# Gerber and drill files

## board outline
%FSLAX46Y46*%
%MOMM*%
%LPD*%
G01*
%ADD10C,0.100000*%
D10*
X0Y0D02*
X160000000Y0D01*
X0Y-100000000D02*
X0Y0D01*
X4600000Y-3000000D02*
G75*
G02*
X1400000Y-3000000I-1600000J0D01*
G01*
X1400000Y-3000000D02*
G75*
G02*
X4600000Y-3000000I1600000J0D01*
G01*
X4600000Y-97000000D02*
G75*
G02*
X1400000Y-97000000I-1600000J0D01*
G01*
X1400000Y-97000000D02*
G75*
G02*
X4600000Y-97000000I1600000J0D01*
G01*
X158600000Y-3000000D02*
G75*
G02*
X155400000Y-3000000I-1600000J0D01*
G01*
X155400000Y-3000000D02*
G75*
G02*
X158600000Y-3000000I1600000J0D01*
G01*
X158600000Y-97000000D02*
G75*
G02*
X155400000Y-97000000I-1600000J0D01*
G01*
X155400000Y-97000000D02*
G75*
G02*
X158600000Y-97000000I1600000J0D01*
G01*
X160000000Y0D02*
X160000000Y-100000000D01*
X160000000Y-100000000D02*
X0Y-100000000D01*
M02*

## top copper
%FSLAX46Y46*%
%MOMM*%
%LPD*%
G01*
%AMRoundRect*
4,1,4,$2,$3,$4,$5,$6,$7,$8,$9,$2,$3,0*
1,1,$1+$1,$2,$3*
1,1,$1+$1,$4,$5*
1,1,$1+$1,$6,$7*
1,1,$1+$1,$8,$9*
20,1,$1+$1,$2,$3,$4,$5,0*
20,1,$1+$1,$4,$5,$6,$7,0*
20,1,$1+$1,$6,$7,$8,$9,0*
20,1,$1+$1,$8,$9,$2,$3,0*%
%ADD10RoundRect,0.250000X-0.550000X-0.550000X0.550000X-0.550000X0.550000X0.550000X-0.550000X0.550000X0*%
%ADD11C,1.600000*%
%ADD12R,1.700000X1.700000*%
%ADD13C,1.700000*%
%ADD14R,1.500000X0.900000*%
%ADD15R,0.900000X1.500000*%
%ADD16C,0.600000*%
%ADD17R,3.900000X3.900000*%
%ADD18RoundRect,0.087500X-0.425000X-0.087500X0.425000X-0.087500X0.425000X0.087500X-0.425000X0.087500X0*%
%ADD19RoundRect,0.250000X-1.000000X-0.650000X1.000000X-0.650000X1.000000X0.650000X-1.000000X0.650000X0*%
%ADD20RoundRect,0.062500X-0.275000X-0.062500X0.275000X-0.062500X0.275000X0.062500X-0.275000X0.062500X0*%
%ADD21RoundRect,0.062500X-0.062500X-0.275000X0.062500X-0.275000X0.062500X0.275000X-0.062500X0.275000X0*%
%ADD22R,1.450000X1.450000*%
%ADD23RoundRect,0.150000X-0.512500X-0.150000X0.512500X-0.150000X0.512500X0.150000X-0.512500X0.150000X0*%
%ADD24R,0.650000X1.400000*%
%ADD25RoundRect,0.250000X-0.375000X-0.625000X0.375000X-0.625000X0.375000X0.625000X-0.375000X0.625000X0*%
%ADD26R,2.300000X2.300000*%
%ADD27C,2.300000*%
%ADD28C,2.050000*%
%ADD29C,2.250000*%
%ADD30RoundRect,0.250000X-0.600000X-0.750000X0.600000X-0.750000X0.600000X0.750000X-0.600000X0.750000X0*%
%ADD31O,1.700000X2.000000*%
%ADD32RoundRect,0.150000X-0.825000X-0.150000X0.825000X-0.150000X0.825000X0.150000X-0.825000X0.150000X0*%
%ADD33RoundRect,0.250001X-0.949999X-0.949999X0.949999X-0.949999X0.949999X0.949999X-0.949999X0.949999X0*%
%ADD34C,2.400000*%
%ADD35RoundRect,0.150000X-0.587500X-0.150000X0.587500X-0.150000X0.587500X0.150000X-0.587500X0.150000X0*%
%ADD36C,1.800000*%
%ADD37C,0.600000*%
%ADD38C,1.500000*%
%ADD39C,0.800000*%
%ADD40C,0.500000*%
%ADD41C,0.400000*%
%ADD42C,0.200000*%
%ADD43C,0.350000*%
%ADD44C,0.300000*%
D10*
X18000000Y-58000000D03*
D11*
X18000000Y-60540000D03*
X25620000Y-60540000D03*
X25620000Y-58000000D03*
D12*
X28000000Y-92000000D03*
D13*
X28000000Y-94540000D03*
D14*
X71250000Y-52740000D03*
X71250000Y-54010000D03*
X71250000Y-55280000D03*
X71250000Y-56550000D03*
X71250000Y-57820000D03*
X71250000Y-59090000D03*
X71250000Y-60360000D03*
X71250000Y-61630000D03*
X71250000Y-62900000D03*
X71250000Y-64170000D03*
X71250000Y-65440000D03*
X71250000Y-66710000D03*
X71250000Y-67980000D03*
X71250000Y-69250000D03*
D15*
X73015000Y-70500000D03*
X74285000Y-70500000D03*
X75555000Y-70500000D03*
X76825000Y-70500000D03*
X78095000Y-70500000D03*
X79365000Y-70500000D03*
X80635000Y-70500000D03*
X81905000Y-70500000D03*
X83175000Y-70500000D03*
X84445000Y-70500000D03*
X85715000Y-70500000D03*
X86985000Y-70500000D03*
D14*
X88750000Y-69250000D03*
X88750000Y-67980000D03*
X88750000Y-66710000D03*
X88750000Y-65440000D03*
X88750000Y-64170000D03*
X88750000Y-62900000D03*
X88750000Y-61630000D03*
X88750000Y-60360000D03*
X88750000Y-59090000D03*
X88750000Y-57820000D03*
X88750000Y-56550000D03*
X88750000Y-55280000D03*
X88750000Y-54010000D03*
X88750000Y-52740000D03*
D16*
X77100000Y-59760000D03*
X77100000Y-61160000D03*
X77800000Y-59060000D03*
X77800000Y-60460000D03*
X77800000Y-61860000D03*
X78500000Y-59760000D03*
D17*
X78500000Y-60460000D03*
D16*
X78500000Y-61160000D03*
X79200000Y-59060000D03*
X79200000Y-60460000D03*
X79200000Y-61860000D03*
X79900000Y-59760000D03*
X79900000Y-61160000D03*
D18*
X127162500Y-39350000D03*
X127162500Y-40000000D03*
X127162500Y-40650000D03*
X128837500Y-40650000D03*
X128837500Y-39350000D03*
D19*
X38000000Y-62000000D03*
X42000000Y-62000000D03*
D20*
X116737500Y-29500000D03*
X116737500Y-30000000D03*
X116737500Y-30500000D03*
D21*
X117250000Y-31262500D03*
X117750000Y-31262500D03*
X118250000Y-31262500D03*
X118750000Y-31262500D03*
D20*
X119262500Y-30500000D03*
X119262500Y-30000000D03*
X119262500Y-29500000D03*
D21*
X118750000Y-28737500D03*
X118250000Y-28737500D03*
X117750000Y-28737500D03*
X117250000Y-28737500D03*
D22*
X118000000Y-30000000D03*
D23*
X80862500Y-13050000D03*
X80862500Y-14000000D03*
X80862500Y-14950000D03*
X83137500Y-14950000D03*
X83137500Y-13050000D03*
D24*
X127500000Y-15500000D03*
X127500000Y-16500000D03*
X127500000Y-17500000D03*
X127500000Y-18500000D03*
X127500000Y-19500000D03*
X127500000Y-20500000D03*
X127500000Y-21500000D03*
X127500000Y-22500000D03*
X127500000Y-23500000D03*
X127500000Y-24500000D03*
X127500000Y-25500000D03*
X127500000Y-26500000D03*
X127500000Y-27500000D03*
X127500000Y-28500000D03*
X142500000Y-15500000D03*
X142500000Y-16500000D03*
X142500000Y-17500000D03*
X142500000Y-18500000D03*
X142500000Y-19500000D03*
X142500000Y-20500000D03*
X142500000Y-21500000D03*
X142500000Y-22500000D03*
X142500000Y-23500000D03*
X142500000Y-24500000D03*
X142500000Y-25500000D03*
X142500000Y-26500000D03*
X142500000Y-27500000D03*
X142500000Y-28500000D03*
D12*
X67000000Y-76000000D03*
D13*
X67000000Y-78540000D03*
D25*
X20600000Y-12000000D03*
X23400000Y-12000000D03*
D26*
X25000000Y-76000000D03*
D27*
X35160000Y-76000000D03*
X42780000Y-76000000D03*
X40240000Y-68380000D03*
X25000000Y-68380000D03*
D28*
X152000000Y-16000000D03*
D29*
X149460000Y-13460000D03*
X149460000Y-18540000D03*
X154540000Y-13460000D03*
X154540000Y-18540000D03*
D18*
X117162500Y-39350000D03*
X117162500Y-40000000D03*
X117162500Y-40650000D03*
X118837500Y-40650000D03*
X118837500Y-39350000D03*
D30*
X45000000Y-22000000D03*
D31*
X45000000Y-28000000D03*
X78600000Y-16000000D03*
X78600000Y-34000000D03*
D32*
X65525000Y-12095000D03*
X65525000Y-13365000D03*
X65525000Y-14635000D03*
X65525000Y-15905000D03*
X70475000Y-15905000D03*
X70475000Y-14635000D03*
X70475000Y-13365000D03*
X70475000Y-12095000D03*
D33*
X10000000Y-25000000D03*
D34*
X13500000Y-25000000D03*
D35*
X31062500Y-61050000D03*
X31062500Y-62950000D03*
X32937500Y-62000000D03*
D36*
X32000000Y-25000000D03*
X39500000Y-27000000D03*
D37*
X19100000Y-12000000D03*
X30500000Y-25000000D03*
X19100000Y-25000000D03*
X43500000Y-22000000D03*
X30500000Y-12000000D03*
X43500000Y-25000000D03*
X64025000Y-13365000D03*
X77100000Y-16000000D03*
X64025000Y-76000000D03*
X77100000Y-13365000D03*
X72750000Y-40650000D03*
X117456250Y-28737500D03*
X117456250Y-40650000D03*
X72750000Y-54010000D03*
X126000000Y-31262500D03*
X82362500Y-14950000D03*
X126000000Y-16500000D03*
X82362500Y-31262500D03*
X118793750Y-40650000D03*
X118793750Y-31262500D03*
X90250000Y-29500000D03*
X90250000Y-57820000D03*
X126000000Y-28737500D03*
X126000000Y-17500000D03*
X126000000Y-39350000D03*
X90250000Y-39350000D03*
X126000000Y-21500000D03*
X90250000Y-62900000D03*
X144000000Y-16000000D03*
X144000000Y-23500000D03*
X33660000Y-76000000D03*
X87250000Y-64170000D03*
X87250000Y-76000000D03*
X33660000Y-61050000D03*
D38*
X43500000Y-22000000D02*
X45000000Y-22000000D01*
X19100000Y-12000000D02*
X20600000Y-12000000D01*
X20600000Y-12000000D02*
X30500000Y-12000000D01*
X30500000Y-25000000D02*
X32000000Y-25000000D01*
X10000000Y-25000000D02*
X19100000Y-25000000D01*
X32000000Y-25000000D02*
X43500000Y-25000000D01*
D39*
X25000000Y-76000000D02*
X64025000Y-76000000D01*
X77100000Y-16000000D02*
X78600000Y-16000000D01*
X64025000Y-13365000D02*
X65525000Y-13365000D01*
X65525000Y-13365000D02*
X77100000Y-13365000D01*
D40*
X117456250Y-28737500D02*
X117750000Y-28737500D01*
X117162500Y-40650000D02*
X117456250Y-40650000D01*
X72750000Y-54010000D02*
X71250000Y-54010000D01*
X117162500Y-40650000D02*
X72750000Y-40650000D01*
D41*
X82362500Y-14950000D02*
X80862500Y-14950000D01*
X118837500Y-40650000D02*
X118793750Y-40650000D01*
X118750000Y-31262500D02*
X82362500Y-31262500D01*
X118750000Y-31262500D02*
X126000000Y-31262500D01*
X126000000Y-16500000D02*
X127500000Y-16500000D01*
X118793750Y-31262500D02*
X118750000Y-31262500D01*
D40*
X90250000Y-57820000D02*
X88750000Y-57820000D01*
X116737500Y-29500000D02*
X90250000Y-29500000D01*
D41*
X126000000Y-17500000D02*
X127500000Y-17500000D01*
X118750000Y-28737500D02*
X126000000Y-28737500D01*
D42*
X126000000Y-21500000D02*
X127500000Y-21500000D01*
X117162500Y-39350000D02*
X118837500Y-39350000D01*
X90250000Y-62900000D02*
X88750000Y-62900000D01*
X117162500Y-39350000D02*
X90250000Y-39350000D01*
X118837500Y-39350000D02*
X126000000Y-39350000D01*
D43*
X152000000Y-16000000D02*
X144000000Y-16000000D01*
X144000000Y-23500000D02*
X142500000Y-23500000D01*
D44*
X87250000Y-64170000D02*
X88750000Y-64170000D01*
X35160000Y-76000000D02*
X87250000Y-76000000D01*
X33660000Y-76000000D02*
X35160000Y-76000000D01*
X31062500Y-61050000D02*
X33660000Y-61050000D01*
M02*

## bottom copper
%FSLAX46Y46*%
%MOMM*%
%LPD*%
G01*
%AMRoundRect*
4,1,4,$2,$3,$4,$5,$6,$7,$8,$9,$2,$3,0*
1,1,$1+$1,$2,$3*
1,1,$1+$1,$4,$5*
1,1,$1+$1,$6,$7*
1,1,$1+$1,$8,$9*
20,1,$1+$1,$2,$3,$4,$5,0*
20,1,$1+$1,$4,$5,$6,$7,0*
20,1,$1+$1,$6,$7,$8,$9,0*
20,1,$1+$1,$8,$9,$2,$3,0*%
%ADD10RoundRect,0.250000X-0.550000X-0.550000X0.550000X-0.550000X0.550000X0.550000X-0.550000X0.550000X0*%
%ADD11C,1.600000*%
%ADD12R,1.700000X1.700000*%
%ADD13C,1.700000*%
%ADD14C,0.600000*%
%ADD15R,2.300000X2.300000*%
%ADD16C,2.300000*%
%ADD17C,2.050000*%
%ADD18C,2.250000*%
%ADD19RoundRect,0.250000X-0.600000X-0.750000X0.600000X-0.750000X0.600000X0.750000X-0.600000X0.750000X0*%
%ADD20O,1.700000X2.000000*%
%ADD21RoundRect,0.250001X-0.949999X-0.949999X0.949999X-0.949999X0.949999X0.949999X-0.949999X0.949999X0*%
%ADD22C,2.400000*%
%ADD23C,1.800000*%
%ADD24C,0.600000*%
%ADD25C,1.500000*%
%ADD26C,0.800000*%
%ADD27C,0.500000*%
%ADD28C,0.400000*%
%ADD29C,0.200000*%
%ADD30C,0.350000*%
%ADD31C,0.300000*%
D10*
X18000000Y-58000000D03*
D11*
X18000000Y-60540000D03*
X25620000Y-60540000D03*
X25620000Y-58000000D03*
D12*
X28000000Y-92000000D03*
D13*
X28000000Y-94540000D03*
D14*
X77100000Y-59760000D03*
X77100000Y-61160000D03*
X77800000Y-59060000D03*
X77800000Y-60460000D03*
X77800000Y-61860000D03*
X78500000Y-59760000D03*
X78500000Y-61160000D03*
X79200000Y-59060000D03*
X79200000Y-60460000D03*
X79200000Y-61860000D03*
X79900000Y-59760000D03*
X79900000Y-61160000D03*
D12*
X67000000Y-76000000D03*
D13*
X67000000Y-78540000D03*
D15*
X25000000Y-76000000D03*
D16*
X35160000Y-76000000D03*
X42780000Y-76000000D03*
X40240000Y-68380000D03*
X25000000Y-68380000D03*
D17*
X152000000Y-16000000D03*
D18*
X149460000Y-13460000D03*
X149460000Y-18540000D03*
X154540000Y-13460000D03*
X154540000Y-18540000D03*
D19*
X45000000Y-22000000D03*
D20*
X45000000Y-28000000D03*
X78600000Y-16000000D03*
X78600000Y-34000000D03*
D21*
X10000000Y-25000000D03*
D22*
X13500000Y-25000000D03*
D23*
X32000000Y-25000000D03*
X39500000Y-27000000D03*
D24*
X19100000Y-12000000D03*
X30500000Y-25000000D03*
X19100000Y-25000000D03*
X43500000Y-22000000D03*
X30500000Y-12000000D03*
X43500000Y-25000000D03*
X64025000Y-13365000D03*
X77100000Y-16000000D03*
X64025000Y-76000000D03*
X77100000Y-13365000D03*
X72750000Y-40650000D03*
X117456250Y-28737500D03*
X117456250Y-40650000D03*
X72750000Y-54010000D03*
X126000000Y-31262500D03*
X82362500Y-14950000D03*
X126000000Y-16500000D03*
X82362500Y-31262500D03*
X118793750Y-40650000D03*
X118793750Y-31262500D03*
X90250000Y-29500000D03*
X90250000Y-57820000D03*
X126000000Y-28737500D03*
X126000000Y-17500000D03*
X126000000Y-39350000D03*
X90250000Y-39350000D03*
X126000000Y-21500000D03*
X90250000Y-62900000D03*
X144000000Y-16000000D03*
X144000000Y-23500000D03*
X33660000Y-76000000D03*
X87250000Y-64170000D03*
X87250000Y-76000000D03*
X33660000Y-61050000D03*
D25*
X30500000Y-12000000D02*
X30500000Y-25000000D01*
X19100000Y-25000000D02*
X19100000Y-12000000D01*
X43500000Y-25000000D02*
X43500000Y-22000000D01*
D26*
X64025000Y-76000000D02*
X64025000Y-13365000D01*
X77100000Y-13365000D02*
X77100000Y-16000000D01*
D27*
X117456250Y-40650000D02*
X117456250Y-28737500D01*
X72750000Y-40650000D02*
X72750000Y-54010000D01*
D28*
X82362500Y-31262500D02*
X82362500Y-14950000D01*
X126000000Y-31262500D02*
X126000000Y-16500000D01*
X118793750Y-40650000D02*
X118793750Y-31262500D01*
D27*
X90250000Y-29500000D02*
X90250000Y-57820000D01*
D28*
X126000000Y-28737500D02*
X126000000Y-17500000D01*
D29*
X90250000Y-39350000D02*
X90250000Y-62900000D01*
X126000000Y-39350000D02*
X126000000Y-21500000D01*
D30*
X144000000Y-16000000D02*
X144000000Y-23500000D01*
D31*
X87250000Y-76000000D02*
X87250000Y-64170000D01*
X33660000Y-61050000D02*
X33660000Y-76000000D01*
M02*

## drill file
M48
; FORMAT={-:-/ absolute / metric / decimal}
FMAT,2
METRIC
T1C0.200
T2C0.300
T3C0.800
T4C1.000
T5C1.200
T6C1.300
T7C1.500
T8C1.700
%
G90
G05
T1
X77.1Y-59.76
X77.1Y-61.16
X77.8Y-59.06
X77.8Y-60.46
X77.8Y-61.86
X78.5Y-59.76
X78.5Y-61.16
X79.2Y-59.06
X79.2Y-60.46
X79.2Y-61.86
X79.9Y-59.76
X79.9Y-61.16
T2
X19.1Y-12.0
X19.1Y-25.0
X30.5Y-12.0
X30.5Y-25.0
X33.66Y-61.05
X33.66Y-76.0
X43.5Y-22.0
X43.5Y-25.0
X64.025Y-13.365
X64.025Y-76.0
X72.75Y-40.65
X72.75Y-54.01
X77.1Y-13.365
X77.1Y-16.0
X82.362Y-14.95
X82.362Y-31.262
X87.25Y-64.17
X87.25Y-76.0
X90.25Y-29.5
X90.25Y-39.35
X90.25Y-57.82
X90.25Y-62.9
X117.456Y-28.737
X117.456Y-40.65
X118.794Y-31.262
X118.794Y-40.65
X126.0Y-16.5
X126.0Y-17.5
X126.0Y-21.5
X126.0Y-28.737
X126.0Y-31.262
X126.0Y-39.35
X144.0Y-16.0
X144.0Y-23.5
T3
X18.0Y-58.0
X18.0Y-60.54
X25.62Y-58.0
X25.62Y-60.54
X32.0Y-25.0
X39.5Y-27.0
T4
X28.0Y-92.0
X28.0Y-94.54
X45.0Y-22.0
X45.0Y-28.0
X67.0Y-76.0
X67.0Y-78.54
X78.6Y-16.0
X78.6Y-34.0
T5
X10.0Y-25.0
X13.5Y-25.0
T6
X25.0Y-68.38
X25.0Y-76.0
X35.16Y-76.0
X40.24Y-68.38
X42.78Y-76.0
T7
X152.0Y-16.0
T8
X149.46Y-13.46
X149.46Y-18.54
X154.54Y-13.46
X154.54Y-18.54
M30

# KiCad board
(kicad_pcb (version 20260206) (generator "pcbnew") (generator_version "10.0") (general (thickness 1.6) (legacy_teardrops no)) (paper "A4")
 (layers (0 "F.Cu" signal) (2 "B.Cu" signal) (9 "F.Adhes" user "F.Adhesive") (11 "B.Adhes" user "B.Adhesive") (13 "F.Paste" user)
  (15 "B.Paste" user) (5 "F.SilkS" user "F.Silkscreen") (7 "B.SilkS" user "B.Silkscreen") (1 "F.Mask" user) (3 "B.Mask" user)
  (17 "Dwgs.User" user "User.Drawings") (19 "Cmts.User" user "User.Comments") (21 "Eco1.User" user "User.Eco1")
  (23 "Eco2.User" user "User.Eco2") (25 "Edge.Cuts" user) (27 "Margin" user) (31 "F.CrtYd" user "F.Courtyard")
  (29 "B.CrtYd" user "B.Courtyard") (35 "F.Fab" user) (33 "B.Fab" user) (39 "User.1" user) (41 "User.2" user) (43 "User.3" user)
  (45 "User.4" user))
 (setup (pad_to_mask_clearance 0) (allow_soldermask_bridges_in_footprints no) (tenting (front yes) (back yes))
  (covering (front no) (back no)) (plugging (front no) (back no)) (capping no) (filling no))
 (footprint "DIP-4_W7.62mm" (layer "F.Cu") (at 18 58)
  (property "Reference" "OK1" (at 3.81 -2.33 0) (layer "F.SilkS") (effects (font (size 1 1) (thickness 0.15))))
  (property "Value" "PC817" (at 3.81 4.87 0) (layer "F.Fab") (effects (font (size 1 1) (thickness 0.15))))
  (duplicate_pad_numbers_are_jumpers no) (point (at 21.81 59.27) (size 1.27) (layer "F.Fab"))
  (pad "1" thru_hole roundrect (at 0 0) (size 1.6 1.6) (drill 0.8) (layers "*.Cu" "*.Mask") (remove_unused_layers no)
   (roundrect_rratio 0.15625))
  (pad "2" thru_hole circle (at 0 2.54) (size 1.6 1.6) (drill 0.8) (layers "*.Cu" "*.Mask") (remove_unused_layers no))
  (pad "3" thru_hole circle (at 7.62 2.54) (size 1.6 1.6) (drill 0.8) (layers "*.Cu" "*.Mask") (remove_unused_layers no))
  (pad "4" thru_hole circle (at 7.62 0) (size 1.6 1.6) (drill 0.8) (layers "*.Cu" "*.Mask") (remove_unused_layers no)))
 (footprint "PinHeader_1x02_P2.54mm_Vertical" (layer "F.Cu") (at 28 92)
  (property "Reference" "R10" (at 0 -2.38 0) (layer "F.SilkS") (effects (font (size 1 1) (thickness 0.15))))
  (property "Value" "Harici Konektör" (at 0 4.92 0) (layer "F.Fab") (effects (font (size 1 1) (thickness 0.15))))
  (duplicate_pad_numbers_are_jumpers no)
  (pad "1" thru_hole rect (at 0 0) (size 1.7 1.7) (drill 1) (layers "*.Cu" "*.Mask") (remove_unused_layers no))
  (pad "2" thru_hole circle (at 0 2.54) (size 1.7 1.7) (drill 1) (layers "*.Cu" "*.Mask") (remove_unused_layers no)))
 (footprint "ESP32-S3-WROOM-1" (layer "F.Cu") (at 80 58)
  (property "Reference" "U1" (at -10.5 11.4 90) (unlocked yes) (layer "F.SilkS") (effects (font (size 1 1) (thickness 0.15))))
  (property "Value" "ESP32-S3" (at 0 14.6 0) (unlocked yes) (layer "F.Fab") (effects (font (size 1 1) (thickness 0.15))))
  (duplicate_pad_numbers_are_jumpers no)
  (pad "" smd rect (at -2.9 1.06) (size 0.9 0.9) (layers "F.Paste"))
  (pad "" smd rect (at -2.9 2.46 270) (size 0.9 0.9) (layers "F.Paste"))
  (pad "" smd rect (at -2.9 3.86) (size 0.9 0.9) (layers "F.Paste"))
  (pad "" smd rect (at -1.5 1.06 270) (size 0.9 0.9) (layers "F.Paste"))
  (pad "" smd rect (at -1.5 2.46 270) (size 0.9 0.9) (layers "F.Paste"))
  (pad "" smd rect (at -1.5 3.86 270) (size 0.9 0.9) (layers "F.Paste"))
  (pad "" smd rect (at -0.1 1.06 270) (size 0.9 0.9) (layers "F.Paste"))
  (pad "" smd rect (at -0.1 2.46 270) (size 0.9 0.9) (layers "F.Paste"))
  (pad "" smd rect (at -0.1 3.86 270) (size 0.9 0.9) (layers "F.Paste"))
  (pad "1" smd rect (at -8.75 -5.26) (size 1.5 0.9) (layers "F.Cu" "F.Mask" "F.Paste"))
  (pad "2" smd rect (at -8.75 -3.99) (size 1.5 0.9) (layers "F.Cu" "F.Mask" "F.Paste") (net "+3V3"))
  (pad "3" smd rect (at -8.75 -2.72) (size 1.5 0.9) (layers "F.Cu" "F.Mask" "F.Paste"))
  (pad "4" smd rect (at -8.75 -1.45) (size 1.5 0.9) (layers "F.Cu" "F.Mask" "F.Paste"))
  (pad "5" smd rect (at -8.75 -0.18) (size 1.5 0.9) (layers "F.Cu" "F.Mask" "F.Paste"))
  (pad "6" smd rect (at -8.75 1.09) (size 1.5 0.9) (layers "F.Cu" "F.Mask" "F.Paste"))
  (pad "7" smd rect (at -8.75 2.36) (size 1.5 0.9) (layers "F.Cu" "F.Mask" "F.Paste"))
  (pad "8" smd rect (at -8.75 3.63) (size 1.5 0.9) (layers "F.Cu" "F.Mask" "F.Paste"))
  (pad "9" smd rect (at -8.75 4.9) (size 1.5 0.9) (layers "F.Cu" "F.Mask" "F.Paste"))
  (pad "10" smd rect (at -8.75 6.17) (size 1.5 0.9) (layers "F.Cu" "F.Mask" "F.Paste"))
  (pad "11" smd rect (at -8.75 7.44) (size 1.5 0.9) (layers "F.Cu" "F.Mask" "F.Paste"))
  (pad "12" smd rect (at -8.75 8.71) (size 1.5 0.9) (layers "F.Cu" "F.Mask" "F.Paste"))
  (pad "13" smd rect (at -8.75 9.98) (size 1.5 0.9) (layers "F.Cu" "F.Mask" "F.Paste"))
  (pad "14" smd rect (at -8.75 11.25 180) (size 1.5 0.9) (layers "F.Cu" "F.Mask" "F.Paste"))
  (pad "15" smd rect (at -6.985 12.5 270) (size 1.5 0.9) (layers "F.Cu" "F.Mask" "F.Paste"))
  (pad "16" smd rect (at -5.715 12.5 270) (size 1.5 0.9) (layers "F.Cu" "F.Mask" "F.Paste"))
  (pad "17" smd rect (at -4.445 12.5 270) (size 1.5 0.9) (layers "F.Cu" "F.Mask" "F.Paste"))
  (pad "18" smd rect (at -3.175 12.5 270) (size 1.5 0.9) (layers "F.Cu" "F.Mask" "F.Paste"))
  (pad "19" smd rect (at -1.905 12.5 270) (size 1.5 0.9) (layers "F.Cu" "F.Mask" "F.Paste"))
  (pad "20" smd rect (at -0.635 12.5 270) (size 1.5 0.9) (layers "F.Cu" "F.Mask" "F.Paste"))
  (pad "21" smd rect (at 0.635 12.5 270) (size 1.5 0.9) (layers "F.Cu" "F.Mask" "F.Paste"))
  (pad "22" smd rect (at 1.905 12.5 270) (size 1.5 0.9) (layers "F.Cu" "F.Mask" "F.Paste"))
  (pad "23" smd rect (at 3.175 12.5 270) (size 1.5 0.9) (layers "F.Cu" "F.Mask" "F.Paste"))
  (pad "24" smd rect (at 4.445 12.5 270) (size 1.5 0.9) (layers "F.Cu" "F.Mask" "F.Paste"))
  (pad "25" smd rect (at 5.715 12.5 270) (size 1.5 0.9) (layers "F.Cu" "F.Mask" "F.Paste"))
  (pad "26" smd rect (at 6.985 12.5 270) (size 1.5 0.9) (layers "F.Cu" "F.Mask" "F.Paste"))
  (pad "27" smd rect (at 8.75 11.25) (size 1.5 0.9) (layers "F.Cu" "F.Mask" "F.Paste"))
  (pad "28" smd rect (at 8.75 9.98) (size 1.5 0.9) (layers "F.Cu" "F.Mask" "F.Paste"))
  (pad "29" smd rect (at 8.75 8.71) (size 1.5 0.9) (layers "F.Cu" "F.Mask" "F.Paste"))
  (pad "30" smd rect (at 8.75 7.44) (size 1.5 0.9) (layers "F.Cu" "F.Mask" "F.Paste"))
  (pad "31" smd rect (at 8.75 6.17) (size 1.5 0.9) (layers "F.Cu" "F.Mask" "F.Paste") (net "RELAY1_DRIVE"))
  (pad "32" smd rect (at 8.75 4.9) (size 1.5 0.9) (layers "F.Cu" "F.Mask" "F.Paste") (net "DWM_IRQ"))
  (pad "33" smd rect (at 8.75 3.63) (size 1.5 0.9) (layers "F.Cu" "F.Mask" "F.Paste"))
  (pad "34" smd rect (at 8.75 2.36) (size 1.5 0.9) (layers "F.Cu" "F.Mask" "F.Paste"))
  (pad "35" smd rect (at 8.75 1.09) (size 1.5 0.9) (layers "F.Cu" "F.Mask" "F.Paste"))
  (pad "36" smd rect (at 8.75 -0.18) (size 1.5 0.9) (layers "F.Cu" "F.Mask" "F.Paste") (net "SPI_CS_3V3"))
  (pad "37" smd rect (at 8.75 -1.45) (size 1.5 0.9) (layers "F.Cu" "F.Mask" "F.Paste"))
  (pad "38" smd rect (at 8.75 -2.72) (size 1.5 0.9) (layers "F.Cu" "F.Mask" "F.Paste"))
  (pad "39" smd rect (at 8.75 -3.99) (size 1.5 0.9) (layers "F.Cu" "F.Mask" "F.Paste"))
  (pad "40" smd rect (at 8.75 -5.26) (size 1.5 0.9) (layers "F.Cu" "F.Mask" "F.Paste"))
  (pad "41" thru_hole circle (at -2.9 1.76 90) (size 0.6 0.6) (drill 0.2) (layers "*.Cu" "F.Mask") (remove_unused_layers no)
   (zone_connect 2))
  (pad "41" thru_hole circle (at -2.9 3.16) (size 0.6 0.6) (drill 0.2) (layers "*.Cu" "F.Mask") (remove_unused_layers no) (zone_connect 2))
  (pad "41" thru_hole circle (at -2.2 1.06) (size 0.6 0.6) (drill 0.2) (layers "*.Cu" "F.Mask") (remove_unused_layers no) (zone_connect 2))
  (pad "41" thru_hole circle (at -2.2 2.46) (size 0.6 0.6) (drill 0.2) (layers "*.Cu" "F.Mask") (remove_unused_layers no) (zone_connect 2))
  (pad "41" thru_hole circle (at -2.2 3.86) (size 0.6 0.6) (drill 0.2) (layers "*.Cu" "F.Mask") (remove_unused_layers no) (zone_connect 2))
  (pad "41" thru_hole circle (at -1.5 1.76) (size 0.6 0.6) (drill 0.2) (layers "*.Cu" "F.Mask") (remove_unused_layers no) (zone_connect 2))
  (pad "41" smd rect (at -1.5 2.46 270) (size 3.9 3.9) (layers "F.Cu" "F.Mask") (zone_connect 2))
  (pad "41" thru_hole circle (at -1.5 3.16) (size 0.6 0.6) (drill 0.2) (layers "*.Cu" "F.Mask") (remove_unused_layers no) (zone_connect 2))
  (pad "41" thru_hole circle (at -0.8 1.06) (size 0.6 0.6) (drill 0.2) (layers "*.Cu" "F.Mask") (remove_unused_layers no) (zone_connect 2))
  (pad "41" thru_hole circle (at -0.8 2.46) (size 0.6 0.6) (drill 0.2) (layers "*.Cu" "F.Mask") (remove_unused_layers no) (zone_connect 2))
  (pad "41" thru_hole circle (at -0.8 3.86) (size 0.6 0.6) (drill 0.2) (layers "*.Cu" "F.Mask") (remove_unused_layers no) (zone_connect 2))
  (pad "41" thru_hole circle (at -0.1 1.76) (size 0.6 0.6) (drill 0.2) (layers "*.Cu" "F.Mask") (remove_unused_layers no) (zone_connect 2))
  (pad "41" thru_hole circle (at -0.1 3.16) (size 0.6 0.6) (drill 0.2) (layers "*.Cu" "F.Mask") (remove_unused_layers no) (zone_connect 2))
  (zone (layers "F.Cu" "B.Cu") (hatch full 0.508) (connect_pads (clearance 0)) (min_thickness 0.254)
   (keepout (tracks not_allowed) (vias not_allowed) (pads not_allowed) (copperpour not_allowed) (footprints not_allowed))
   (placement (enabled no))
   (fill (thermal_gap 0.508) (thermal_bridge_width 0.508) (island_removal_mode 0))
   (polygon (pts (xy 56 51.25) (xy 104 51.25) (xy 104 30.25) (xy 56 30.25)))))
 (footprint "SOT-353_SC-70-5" (layer "F.Cu") (at 128 40)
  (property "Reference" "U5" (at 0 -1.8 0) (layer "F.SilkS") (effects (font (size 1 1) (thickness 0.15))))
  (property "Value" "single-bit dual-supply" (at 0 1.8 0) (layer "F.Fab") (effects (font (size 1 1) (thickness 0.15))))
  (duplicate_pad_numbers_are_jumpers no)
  (pad "1" smd roundrect (at -0.8375 -0.65) (size 1.025 0.35) (layers "F.Cu" "F.Mask" "F.Paste") (roundrect_rratio 0.25))
  (pad "2" smd roundrect (at -0.8375 0) (size 1.025 0.35) (layers "F.Cu" "F.Mask" "F.Paste") (roundrect_rratio 0.25))
  (pad "3" smd roundrect (at -0.8375 0.65) (size 1.025 0.35) (layers "F.Cu" "F.Mask" "F.Paste") (roundrect_rratio 0.25))
  (pad "4" smd roundrect (at 0.8375 0.65) (size 1.025 0.35) (layers "F.Cu" "F.Mask" "F.Paste") (roundrect_rratio 0.25))
  (pad "5" smd roundrect (at 0.8375 -0.65) (size 1.025 0.35) (layers "F.Cu" "F.Mask" "F.Paste") (roundrect_rratio 0.25)))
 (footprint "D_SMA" (layer "F.Cu") (at 40 62)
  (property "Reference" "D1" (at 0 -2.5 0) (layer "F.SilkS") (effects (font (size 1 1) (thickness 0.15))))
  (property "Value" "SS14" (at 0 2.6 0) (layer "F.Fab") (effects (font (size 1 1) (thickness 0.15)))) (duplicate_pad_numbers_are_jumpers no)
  (pad "1" smd roundrect (at -2 0) (size 2.5 1.8) (layers "F.Cu" "F.Mask" "F.Paste") (roundrect_rratio 0.1388888889))
  (pad "2" smd roundrect (at 2 0) (size 2.5 1.8) (layers "F.Cu" "F.Mask" "F.Paste") (roundrect_rratio 0.1388888889)))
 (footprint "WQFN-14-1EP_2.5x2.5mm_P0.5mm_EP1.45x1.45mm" (layer "F.Cu") (at 118 30)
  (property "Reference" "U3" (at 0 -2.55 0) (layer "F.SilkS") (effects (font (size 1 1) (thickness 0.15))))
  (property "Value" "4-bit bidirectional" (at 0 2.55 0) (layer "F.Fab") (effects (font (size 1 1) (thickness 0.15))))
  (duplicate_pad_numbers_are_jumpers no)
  (pad "" smd roundrect (at -0.36 -0.36) (size 0.58 0.58) (layers "F.Paste") (roundrect_rratio 0.25))
  (pad "" smd roundrect (at -0.36 0.36) (size 0.58 0.58) (layers "F.Paste") (roundrect_rratio 0.25))
  (pad "" smd roundrect (at 0.36 -0.36) (size 0.58 0.58) (layers "F.Paste") (roundrect_rratio 0.25))
  (pad "" smd roundrect (at 0.36 0.36) (size 0.58 0.58) (layers "F.Paste") (roundrect_rratio 0.25))
  (pad "1" smd roundrect (at -1.2625 -0.5) (size 0.675 0.25) (layers "F.Cu" "F.Mask" "F.Paste") (roundrect_rratio 0.25) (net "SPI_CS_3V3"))
  (pad "2" smd roundrect (at -1.2625 0) (size 0.675 0.25) (layers "F.Cu" "F.Mask" "F.Paste") (roundrect_rratio 0.25))
  (pad "3" smd roundrect (at -1.2625 0.5) (size 0.675 0.25) (layers "F.Cu" "F.Mask" "F.Paste") (roundrect_rratio 0.25))
  (pad "4" smd roundrect (at -0.75 1.2625) (size 0.25 0.675) (layers "F.Cu" "F.Mask" "F.Paste") (roundrect_rratio 0.25))
  (pad "5" smd roundrect (at -0.25 1.2625) (size 0.25 0.675) (layers "F.Cu" "F.Mask" "F.Paste") (roundrect_rratio 0.25))
  (pad "6" smd roundrect (at 0.25 1.2625) (size 0.25 0.675) (layers "F.Cu" "F.Mask" "F.Paste") (roundrect_rratio 0.25))
  (pad "7" smd roundrect (at 0.75 1.2625) (size 0.25 0.675) (layers "F.Cu" "F.Mask" "F.Paste") (roundrect_rratio 0.25) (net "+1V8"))
  (pad "8" smd roundrect (at 1.2625 0.5) (size 0.675 0.25) (layers "F.Cu" "F.Mask" "F.Paste") (roundrect_rratio 0.25))
  (pad "9" smd roundrect (at 1.2625 0) (size 0.675 0.25) (layers "F.Cu" "F.Mask" "F.Paste") (roundrect_rratio 0.25))
  (pad "10" smd roundrect (at 1.2625 -0.5) (size 0.675 0.25) (layers "F.Cu" "F.Mask" "F.Paste") (roundrect_rratio 0.25))
  (pad "11" smd roundrect (at 0.75 -1.2625) (size 0.25 0.675) (layers "F.Cu" "F.Mask" "F.Paste") (roundrect_rratio 0.25) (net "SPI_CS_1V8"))
  (pad "12" smd roundrect (at 0.25 -1.2625) (size 0.25 0.675) (layers "F.Cu" "F.Mask" "F.Paste") (roundrect_rratio 0.25))
  (pad "13" smd roundrect (at -0.25 -1.2625) (size 0.25 0.675) (layers "F.Cu" "F.Mask" "F.Paste") (roundrect_rratio 0.25) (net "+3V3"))
  (pad "14" smd roundrect (at -0.75 -1.2625) (size 0.25 0.675) (layers "F.Cu" "F.Mask" "F.Paste") (roundrect_rratio 0.25))
  (pad "15" smd rect (at 0 0) (size 1.45 1.45) (layers "F.Cu" "F.Mask") (zone_connect 2)))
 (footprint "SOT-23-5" (layer "F.Cu") (at 82 14)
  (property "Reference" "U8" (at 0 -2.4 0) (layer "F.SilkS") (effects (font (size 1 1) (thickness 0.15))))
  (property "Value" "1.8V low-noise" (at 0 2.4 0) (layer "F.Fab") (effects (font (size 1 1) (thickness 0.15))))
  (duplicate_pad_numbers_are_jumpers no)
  (pad "1" smd roundrect (at -1.1375 -0.95) (size 1.325 0.6) (layers "F.Cu" "F.Mask" "F.Paste") (roundrect_rratio 0.25))
  (pad "2" smd roundrect (at -1.1375 0) (size 1.325 0.6) (layers "F.Cu" "F.Mask" "F.Paste") (roundrect_rratio 0.25))
  (pad "3" smd roundrect (at -1.1375 0.95) (size 1.325 0.6) (layers "F.Cu" "F.Mask" "F.Paste") (roundrect_rratio 0.25) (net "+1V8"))
  (pad "4" smd roundrect (at 1.1375 0.95) (size 1.325 0.6) (layers "F.Cu" "F.Mask" "F.Paste") (roundrect_rratio 0.25))
  (pad "5" smd roundrect (at 1.1375 -0.95) (size 1.325 0.6) (layers "F.Cu" "F.Mask" "F.Paste") (roundrect_rratio 0.25)))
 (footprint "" (layer "F.Cu") (at 135 22)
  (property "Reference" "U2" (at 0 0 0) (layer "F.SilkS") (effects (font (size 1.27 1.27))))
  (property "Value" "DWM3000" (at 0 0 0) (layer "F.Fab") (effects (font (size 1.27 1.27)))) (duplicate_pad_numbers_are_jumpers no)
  (pad "1" smd rect (at -7.5 -6.5) (size 0.65 1.4) (layers "F.Cu" "F.Mask" "F.Paste") (thermal_bridge_angle 45))
  (pad "2" smd rect (at -7.5 -5.5) (size 0.65 1.4) (layers "F.Cu" "F.Mask" "F.Paste") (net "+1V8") (thermal_bridge_angle 45))
  (pad "3" smd rect (at -7.5 -4.5) (size 0.65 1.4) (layers "F.Cu" "F.Mask" "F.Paste") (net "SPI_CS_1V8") (thermal_bridge_angle 45))
  (pad "4" smd rect (at -7.5 -3.5) (size 0.65 1.4) (layers "F.Cu" "F.Mask" "F.Paste") (thermal_bridge_angle 45))
  (pad "5" smd rect (at -7.5 -2.5) (size 0.65 1.4) (layers "F.Cu" "F.Mask" "F.Paste") (thermal_bridge_angle 45))
  (pad "6" smd rect (at -7.5 -1.5) (size 0.65 1.4) (layers "F.Cu" "F.Mask" "F.Paste") (thermal_bridge_angle 45))
  (pad "7" smd rect (at -7.5 -0.5) (size 0.65 1.4) (layers "F.Cu" "F.Mask" "F.Paste") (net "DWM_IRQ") (thermal_bridge_angle 45))
  (pad "8" smd rect (at -7.5 0.5) (size 0.65 1.4) (layers "F.Cu" "F.Mask" "F.Paste") (thermal_bridge_angle 45))
  (pad "9" smd rect (at -7.5 1.5) (size 0.65 1.4) (layers "F.Cu" "F.Mask" "F.Paste") (thermal_bridge_angle 45))
  (pad "10" smd rect (at -7.5 2.5) (size 0.65 1.4) (layers "F.Cu" "F.Mask" "F.Paste") (thermal_bridge_angle 45))
  (pad "11" smd rect (at -7.5 3.5) (size 0.65 1.4) (layers "F.Cu" "F.Mask" "F.Paste") (thermal_bridge_angle 45))
  (pad "12" smd rect (at -7.5 4.5) (size 0.65 1.4) (layers "F.Cu" "F.Mask" "F.Paste") (thermal_bridge_angle 45))
  (pad "13" smd rect (at -7.5 5.5) (size 0.65 1.4) (layers "F.Cu" "F.Mask" "F.Paste") (thermal_bridge_angle 45))
  (pad "14" smd rect (at -7.5 6.5) (size 0.65 1.4) (layers "F.Cu" "F.Mask" "F.Paste") (thermal_bridge_angle 45))
  (pad "15" smd rect (at 7.5 -6.5) (size 0.65 1.4) (layers "F.Cu" "F.Mask" "F.Paste") (thermal_bridge_angle 45))
  (pad "16" smd rect (at 7.5 -5.5) (size 0.65 1.4) (layers "F.Cu" "F.Mask" "F.Paste") (thermal_bridge_angle 45))
  (pad "17" smd rect (at 7.5 -4.5) (size 0.65 1.4) (layers "F.Cu" "F.Mask" "F.Paste") (thermal_bridge_angle 45))
  (pad "18" smd rect (at 7.5 -3.5) (size 0.65 1.4) (layers "F.Cu" "F.Mask" "F.Paste") (thermal_bridge_angle 45))
  (pad "19" smd rect (at 7.5 -2.5) (size 0.65 1.4) (layers "F.Cu" "F.Mask" "F.Paste") (thermal_bridge_angle 45))
  (pad "20" smd rect (at 7.5 -1.5) (size 0.65 1.4) (layers "F.Cu" "F.Mask" "F.Paste") (thermal_bridge_angle 45))
  (pad "21" smd rect (at 7.5 -0.5) (size 0.65 1.4) (layers "F.Cu" "F.Mask" "F.Paste") (thermal_bridge_angle 45))
  (pad "22" smd rect (at 7.5 0.5) (size 0.65 1.4) (layers "F.Cu" "F.Mask" "F.Paste") (thermal_bridge_angle 45))
  (pad "23" smd rect (at 7.5 1.5) (size 0.65 1.4) (layers "F.Cu" "F.Mask" "F.Paste") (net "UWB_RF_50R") (thermal_bridge_angle 45))
  (pad "24" smd rect (at 7.5 2.5) (size 0.65 1.4) (layers "F.Cu" "F.Mask" "F.Paste") (thermal_bridge_angle 45))
  (pad "25" smd rect (at 7.5 3.5) (size 0.65 1.4) (layers "F.Cu" "F.Mask" "F.Paste") (thermal_bridge_angle 45))
  (pad "26" smd rect (at 7.5 4.5) (size 0.65 1.4) (layers "F.Cu" "F.Mask" "F.Paste") (thermal_bridge_angle 45))
  (pad "27" smd rect (at 7.5 5.5) (size 0.65 1.4) (layers "F.Cu" "F.Mask" "F.Paste") (thermal_bridge_angle 45))
  (pad "28" smd rect (at 7.5 6.5) (size 0.65 1.4) (layers "F.Cu" "F.Mask" "F.Paste") (thermal_bridge_angle 45)))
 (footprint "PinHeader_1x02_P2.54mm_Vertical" (layer "F.Cu") (at 67 76)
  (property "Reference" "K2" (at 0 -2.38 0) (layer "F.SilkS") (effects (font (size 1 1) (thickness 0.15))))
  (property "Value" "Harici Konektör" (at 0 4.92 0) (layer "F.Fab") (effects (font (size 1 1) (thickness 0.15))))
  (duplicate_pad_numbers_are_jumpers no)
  (pad "1" thru_hole rect (at 0 0) (size 1.7 1.7) (drill 1) (layers "*.Cu" "*.Mask") (remove_unused_layers no))
  (pad "2" thru_hole circle (at 0 2.54) (size 1.7 1.7) (drill 1) (layers "*.Cu" "*.Mask") (remove_unused_layers no)))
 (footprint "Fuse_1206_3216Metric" (layer "F.Cu") (at 22 12)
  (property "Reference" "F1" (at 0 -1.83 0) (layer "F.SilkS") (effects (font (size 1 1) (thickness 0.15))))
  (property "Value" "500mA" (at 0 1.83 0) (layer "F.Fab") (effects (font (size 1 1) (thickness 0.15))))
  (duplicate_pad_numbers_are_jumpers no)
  (pad "1" smd roundrect (at -1.4 0) (size 1.25 1.75) (layers "F.Cu" "F.Mask" "F.Paste") (roundrect_rratio 0.2) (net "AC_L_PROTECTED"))
  (pad "2" smd roundrect (at 1.4 0) (size 1.25 1.75) (layers "F.Cu" "F.Mask" "F.Paste") (roundrect_rratio 0.2)))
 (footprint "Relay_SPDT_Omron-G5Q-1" (layer "F.Cu") (at 25 76)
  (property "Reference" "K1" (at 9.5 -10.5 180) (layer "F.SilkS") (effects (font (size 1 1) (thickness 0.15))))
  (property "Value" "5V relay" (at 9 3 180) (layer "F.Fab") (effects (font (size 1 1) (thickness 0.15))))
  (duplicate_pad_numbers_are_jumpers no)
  (pad "1" thru_hole rect (at 0 0 180) (size 2.3 2.3) (drill 1.3) (layers "*.Cu" "*.Mask") (remove_unused_layers no) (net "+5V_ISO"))
  (pad "2" thru_hole circle (at 10.16 0 180) (size 2.3 2.3) (drill 1.3) (layers "*.Cu" "*.Mask") (remove_unused_layers no)
   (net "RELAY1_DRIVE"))
  (pad "3" thru_hole circle (at 17.78 0 180) (size 2.3 2.3) (drill 1.3) (layers "*.Cu" "*.Mask") (remove_unused_layers no))
  (pad "4" thru_hole circle (at 15.24 -7.62 180) (size 2.3 2.3) (drill 1.3) (layers "*.Cu" "*.Mask") (remove_unused_layers no))
  (pad "5" thru_hole circle (at 0 -7.62 180) (size 2.3 2.3) (drill 1.3) (layers "*.Cu" "*.Mask") (remove_unused_layers no)))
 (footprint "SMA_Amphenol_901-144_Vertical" (layer "F.Cu") (at 152 16)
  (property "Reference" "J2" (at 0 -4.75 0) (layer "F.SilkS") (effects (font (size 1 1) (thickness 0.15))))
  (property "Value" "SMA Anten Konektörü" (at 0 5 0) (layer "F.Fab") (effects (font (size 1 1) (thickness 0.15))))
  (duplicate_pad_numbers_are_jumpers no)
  (pad "1" thru_hole circle (at 0 0) (size 2.05 2.05) (drill 1.5) (layers "*.Cu" "*.Mask") (remove_unused_layers no) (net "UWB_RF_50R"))
  (pad "2" thru_hole circle (at -2.54 -2.54) (size 2.25 2.25) (drill 1.7) (layers "*.Cu" "*.Mask") (remove_unused_layers no))
  (pad "2" thru_hole circle (at -2.54 2.54) (size 2.25 2.25) (drill 1.7) (layers "*.Cu" "*.Mask") (remove_unused_layers no))
  (pad "2" thru_hole circle (at 2.54 -2.54) (size 2.25 2.25) (drill 1.7) (layers "*.Cu" "*.Mask") (remove_unused_layers no))
  (pad "2" thru_hole circle (at 2.54 2.54) (size 2.25 2.25) (drill 1.7) (layers "*.Cu" "*.Mask") (remove_unused_layers no)))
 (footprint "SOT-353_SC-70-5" (layer "F.Cu") (at 118 40)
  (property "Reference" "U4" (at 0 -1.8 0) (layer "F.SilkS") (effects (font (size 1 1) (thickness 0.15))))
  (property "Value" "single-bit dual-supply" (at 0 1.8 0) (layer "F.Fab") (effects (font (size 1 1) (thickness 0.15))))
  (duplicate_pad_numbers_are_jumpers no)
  (pad "1" smd roundrect (at -0.8375 -0.65) (size 1.025 0.35) (layers "F.Cu" "F.Mask" "F.Paste") (roundrect_rratio 0.25) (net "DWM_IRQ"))
  (pad "2" smd roundrect (at -0.8375 0) (size 1.025 0.35) (layers "F.Cu" "F.Mask" "F.Paste") (roundrect_rratio 0.25))
  (pad "3" smd roundrect (at -0.8375 0.65) (size 1.025 0.35) (layers "F.Cu" "F.Mask" "F.Paste") (roundrect_rratio 0.25) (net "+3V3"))
  (pad "4" smd roundrect (at 0.8375 0.65) (size 1.025 0.35) (layers "F.Cu" "F.Mask" "F.Paste") (roundrect_rratio 0.25) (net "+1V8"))
  (pad "5" smd roundrect (at 0.8375 -0.65) (size 1.025 0.35) (layers "F.Cu" "F.Mask" "F.Paste") (roundrect_rratio 0.25) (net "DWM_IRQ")))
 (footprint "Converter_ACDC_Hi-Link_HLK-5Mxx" (layer "F.Cu") (at 45 22)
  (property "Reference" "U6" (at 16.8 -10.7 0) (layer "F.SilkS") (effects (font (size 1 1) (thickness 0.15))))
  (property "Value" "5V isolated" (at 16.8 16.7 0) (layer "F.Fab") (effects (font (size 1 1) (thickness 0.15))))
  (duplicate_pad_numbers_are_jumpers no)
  (pad "1" thru_hole roundrect (at 0 0) (size 1.7 2) (drill 1) (layers "*.Cu" "*.Mask") (remove_unused_layers no)
   (roundrect_rratio 0.147059) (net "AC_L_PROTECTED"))
  (pad "2" thru_hole oval (at 0 6) (size 1.7 2) (drill 1) (layers "*.Cu" "*.Mask") (remove_unused_layers no))
  (pad "3" thru_hole oval (at 33.6 -6) (size 1.7 2) (drill 1) (layers "*.Cu" "*.Mask") (remove_unused_layers no) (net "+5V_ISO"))
  (pad "4" thru_hole oval (at 33.6 12) (size 1.7 2) (drill 1) (layers "*.Cu" "*.Mask") (remove_unused_layers no)))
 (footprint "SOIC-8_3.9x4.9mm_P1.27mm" (layer "F.Cu") (at 68 14)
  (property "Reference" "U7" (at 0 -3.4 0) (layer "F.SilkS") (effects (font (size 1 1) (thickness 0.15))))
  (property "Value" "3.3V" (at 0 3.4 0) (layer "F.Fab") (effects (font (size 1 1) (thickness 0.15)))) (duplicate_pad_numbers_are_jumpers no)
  (pad "1" smd roundrect (at -2.475 -1.905) (size 1.95 0.6) (layers "F.Cu" "F.Mask" "F.Paste") (roundrect_rratio 0.25))
  (pad "2" smd roundrect (at -2.475 -0.635) (size 1.95 0.6) (layers "F.Cu" "F.Mask" "F.Paste") (roundrect_rratio 0.25) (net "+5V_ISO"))
  (pad "3" smd roundrect (at -2.475 0.635) (size 1.95 0.6) (layers "F.Cu" "F.Mask" "F.Paste") (roundrect_rratio 0.25))
  (pad "4" smd roundrect (at -2.475 1.905) (size 1.95 0.6) (layers "F.Cu" "F.Mask" "F.Paste") (roundrect_rratio 0.25))
  (pad "5" smd roundrect (at 2.475 1.905) (size 1.95 0.6) (layers "F.Cu" "F.Mask" "F.Paste") (roundrect_rratio 0.25))
  (pad "6" smd roundrect (at 2.475 0.635) (size 1.95 0.6) (layers "F.Cu" "F.Mask" "F.Paste") (roundrect_rratio 0.25))
  (pad "7" smd roundrect (at 2.475 -0.635) (size 1.95 0.6) (layers "F.Cu" "F.Mask" "F.Paste") (roundrect_rratio 0.25))
  (pad "8" smd roundrect (at 2.475 -1.905) (size 1.95 0.6) (layers "F.Cu" "F.Mask" "F.Paste") (roundrect_rratio 0.25)))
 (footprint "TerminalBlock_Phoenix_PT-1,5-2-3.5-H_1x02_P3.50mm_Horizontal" (layer "F.Cu") (at 10 25)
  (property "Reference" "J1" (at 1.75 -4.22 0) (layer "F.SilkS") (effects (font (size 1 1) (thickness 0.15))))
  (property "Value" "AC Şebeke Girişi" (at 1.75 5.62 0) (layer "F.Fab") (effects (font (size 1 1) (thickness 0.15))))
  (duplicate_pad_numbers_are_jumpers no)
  (pad "1" thru_hole roundrect (at 0 0) (size 2.4 2.4) (drill 1.2) (layers "*.Cu" "*.Mask") (remove_unused_layers no)
   (roundrect_rratio 0.104167) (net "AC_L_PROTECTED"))
  (pad "2" thru_hole circle (at 3.5 0) (size 2.4 2.4) (drill 1.2) (layers "*.Cu" "*.Mask") (remove_unused_layers no)))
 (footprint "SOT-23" (layer "F.Cu") (at 32 62)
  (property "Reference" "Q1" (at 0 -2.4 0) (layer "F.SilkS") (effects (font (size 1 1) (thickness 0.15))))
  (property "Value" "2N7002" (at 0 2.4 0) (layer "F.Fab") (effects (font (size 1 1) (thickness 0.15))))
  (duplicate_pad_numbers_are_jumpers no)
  (pad "1" smd roundrect (at -0.9375 -0.95) (size 1.475 0.6) (layers "F.Cu" "F.Mask" "F.Paste") (roundrect_rratio 0.25) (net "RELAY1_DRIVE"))
  (pad "2" smd roundrect (at -0.9375 0.95) (size 1.475 0.6) (layers "F.Cu" "F.Mask" "F.Paste") (roundrect_rratio 0.25))
  (pad "3" smd roundrect (at 0.9375 0) (size 1.475 0.6) (layers "F.Cu" "F.Mask" "F.Paste") (roundrect_rratio 0.25)))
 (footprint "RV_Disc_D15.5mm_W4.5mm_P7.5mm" (layer "F.Cu") (at 32 25)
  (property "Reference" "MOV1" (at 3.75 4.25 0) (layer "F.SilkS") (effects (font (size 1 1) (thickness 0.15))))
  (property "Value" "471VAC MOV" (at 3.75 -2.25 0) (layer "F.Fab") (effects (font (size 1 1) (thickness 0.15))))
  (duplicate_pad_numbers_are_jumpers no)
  (pad "1" thru_hole circle (at 0 0) (size 1.8 1.8) (drill 0.8) (layers "*.Cu" "*.Mask") (remove_unused_layers no) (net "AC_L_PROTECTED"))
  (pad "2" thru_hole circle (at 7.5 2) (size 1.8 1.8) (drill 0.8) (layers "*.Cu" "*.Mask") (remove_unused_layers no)))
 (gr_line (start 0 0) (end 160 0) (stroke (width 0.1) (type default)) (layer "Edge.Cuts"))
 (gr_line (start 0 100) (end 0 0) (stroke (width 0.1) (type default)) (layer "Edge.Cuts"))
 (gr_circle (center 3 3) (end 4.6 3) (stroke (width 0.1) (type default)) (fill no) (layer "Edge.Cuts"))
 (gr_circle (center 3 97) (end 4.6 97) (stroke (width 0.1) (type default)) (fill no) (layer "Edge.Cuts"))
 (gr_circle (center 157 3) (end 158.6 3) (stroke (width 0.1) (type default)) (fill no) (layer "Edge.Cuts"))
 (gr_circle (center 157 97) (end 158.6 97) (stroke (width 0.1) (type default)) (fill no) (layer "Edge.Cuts"))
 (gr_line (start 160 0) (end 160 100) (stroke (width 0.1) (type default)) (layer "Edge.Cuts"))
 (gr_line (start 160 100) (end 0 100) (stroke (width 0.1) (type default)) (layer "Edge.Cuts"))
 (segment (start 43.5 22) (end 45 22) (width 1.5) (layer "F.Cu") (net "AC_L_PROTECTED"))
 (segment (start 19.1 12) (end 20.6 12) (width 1.5) (layer "F.Cu") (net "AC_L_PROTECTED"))
 (segment (start 20.6 12) (end 30.5 12) (width 1.5) (layer "F.Cu") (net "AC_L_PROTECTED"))
 (segment (start 30.5 25) (end 32 25) (width 1.5) (layer "F.Cu") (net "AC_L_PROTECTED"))
 (segment (start 10 25) (end 19.1 25) (width 1.5) (layer "F.Cu") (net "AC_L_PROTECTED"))
 (segment (start 32 25) (end 43.5 25) (width 1.5) (layer "F.Cu") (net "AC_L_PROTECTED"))
 (via (at 19.1 12) (size 0.6) (drill 0.3) (layers "F.Cu" "B.Cu") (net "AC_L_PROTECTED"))
 (via (at 30.5 25) (size 0.6) (drill 0.3) (layers "F.Cu" "B.Cu") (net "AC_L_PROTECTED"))
 (via (at 19.1 25) (size 0.6) (drill 0.3) (layers "F.Cu" "B.Cu") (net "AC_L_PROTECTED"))
 (via (at 43.5 22) (size 0.6) (drill 0.3) (layers "F.Cu" "B.Cu") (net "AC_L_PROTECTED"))
 (via (at 30.5 12) (size 0.6) (drill 0.3) (layers "F.Cu" "B.Cu") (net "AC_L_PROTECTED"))
 (via (at 43.5 25) (size 0.6) (drill 0.3) (layers "F.Cu" "B.Cu") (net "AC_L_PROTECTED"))
 (segment (start 30.5 12) (end 30.5 25) (width 1.5) (layer "B.Cu") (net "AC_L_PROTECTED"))
 (segment (start 19.1 25) (end 19.1 12) (width 1.5) (layer "B.Cu") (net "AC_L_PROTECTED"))
 (segment (start 43.5 25) (end 43.5 22) (width 1.5) (layer "B.Cu") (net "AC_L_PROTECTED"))
 (segment (start 25 76) (end 64.025 76) (width 0.8) (layer "F.Cu") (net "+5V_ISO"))
 (segment (start 77.1 16) (end 78.6 16) (width 0.8) (layer "F.Cu") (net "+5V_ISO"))
 (segment (start 64.025 13.365) (end 65.525 13.365) (width 0.8) (layer "F.Cu") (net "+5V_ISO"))
 (segment (start 65.525 13.365) (end 77.1 13.365) (width 0.8) (layer "F.Cu") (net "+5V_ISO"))
 (via (at 64.025 13.365) (size 0.6) (drill 0.3) (layers "F.Cu" "B.Cu") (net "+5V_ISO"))
 (via (at 77.1 16) (size 0.6) (drill 0.3) (layers "F.Cu" "B.Cu") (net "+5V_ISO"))
 (via (at 64.025 76) (size 0.6) (drill 0.3) (layers "F.Cu" "B.Cu") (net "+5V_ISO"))
 (via (at 77.1 13.365) (size 0.6) (drill 0.3) (layers "F.Cu" "B.Cu") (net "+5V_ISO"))
 (segment (start 64.025 76) (end 64.025 13.365) (width 0.8) (layer "B.Cu") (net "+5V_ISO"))
 (segment (start 77.1 13.365) (end 77.1 16) (width 0.8) (layer "B.Cu") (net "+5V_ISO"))
 (segment (start 117.45625 28.7375) (end 117.75 28.7375) (width 0.5) (layer "F.Cu") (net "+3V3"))
 (segment (start 117.1625 40.65) (end 117.45625 40.65) (width 0.5) (layer "F.Cu") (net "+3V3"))
 (segment (start 72.75 54.01) (end 71.25 54.01) (width 0.5) (layer "F.Cu") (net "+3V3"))
 (segment (start 117.1625 40.65) (end 72.75 40.65) (width 0.5) (layer "F.Cu") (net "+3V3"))
 (via (at 72.75 40.65) (size 0.6) (drill 0.3) (layers "F.Cu" "B.Cu") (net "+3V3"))
 (via (at 117.45625 28.7375) (size 0.6) (drill 0.3) (layers "F.Cu" "B.Cu") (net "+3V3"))
 (via (at 117.45625 40.65) (size 0.6) (drill 0.3) (layers "F.Cu" "B.Cu") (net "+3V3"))
 (via (at 72.75 54.01) (size 0.6) (drill 0.3) (layers "F.Cu" "B.Cu") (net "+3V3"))
 (segment (start 117.45625 40.65) (end 117.45625 28.7375) (width 0.5) (layer "B.Cu") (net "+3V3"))
 (segment (start 72.75 40.65) (end 72.75 54.01) (width 0.5) (layer "B.Cu") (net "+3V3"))
 (segment (start 82.3625 14.95) (end 80.8625 14.95) (width 0.4) (layer "F.Cu") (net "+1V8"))
 (segment (start 118.8375 40.65) (end 118.79375 40.65) (width 0.4) (layer "F.Cu") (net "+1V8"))
 (segment (start 118.75 31.2625) (end 82.3625 31.2625) (width 0.4) (layer "F.Cu") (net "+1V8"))
 (segment (start 118.75 31.2625) (end 126 31.2625) (width 0.4) (layer "F.Cu") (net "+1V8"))
 (segment (start 126 16.5) (end 127.5 16.5) (width 0.4) (layer "F.Cu") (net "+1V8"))
 (segment (start 118.79375 31.2625) (end 118.75 31.2625) (width 0.4) (layer "F.Cu") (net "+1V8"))
 (via (at 126 31.2625) (size 0.6) (drill 0.3) (layers "F.Cu" "B.Cu") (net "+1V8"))
 (via (at 82.3625 14.95) (size 0.6) (drill 0.3) (layers "F.Cu" "B.Cu") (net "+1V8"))
 (via (at 126 16.5) (size 0.6) (drill 0.3) (layers "F.Cu" "B.Cu") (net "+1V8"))
 (via (at 82.3625 31.2625) (size 0.6) (drill 0.3) (layers "F.Cu" "B.Cu") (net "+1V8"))
 (via (at 118.79375 40.65) (size 0.6) (drill 0.3) (layers "F.Cu" "B.Cu") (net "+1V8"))
 (via (at 118.79375 31.2625) (size 0.6) (drill 0.3) (layers "F.Cu" "B.Cu") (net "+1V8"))
 (segment (start 82.3625 31.2625) (end 82.3625 14.95) (width 0.4) (layer "B.Cu") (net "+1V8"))
 (segment (start 126 31.2625) (end 126 16.5) (width 0.4) (layer "B.Cu") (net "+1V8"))
 (segment (start 118.79375 40.65) (end 118.79375 31.2625) (width 0.4) (layer "B.Cu") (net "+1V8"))
 (segment (start 90.25 57.82) (end 88.75 57.82) (width 0.5) (layer "F.Cu") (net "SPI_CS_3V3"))
 (segment (start 116.7375 29.5) (end 90.25 29.5) (width 0.5) (layer "F.Cu") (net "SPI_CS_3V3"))
 (via (at 90.25 29.5) (size 0.6) (drill 0.3) (layers "F.Cu" "B.Cu") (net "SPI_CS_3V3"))
 (via (at 90.25 57.82) (size 0.6) (drill 0.3) (layers "F.Cu" "B.Cu") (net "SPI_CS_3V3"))
 (segment (start 90.25 29.5) (end 90.25 57.82) (width 0.5) (layer "B.Cu") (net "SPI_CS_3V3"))
 (segment (start 126 17.5) (end 127.5 17.5) (width 0.4) (layer "F.Cu") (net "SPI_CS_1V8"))
 (segment (start 118.75 28.7375) (end 126 28.7375) (width 0.4) (layer "F.Cu") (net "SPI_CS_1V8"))
 (via (at 126 28.7375) (size 0.6) (drill 0.3) (layers "F.Cu" "B.Cu") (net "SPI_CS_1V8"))
 (via (at 126 17.5) (size 0.6) (drill 0.3) (layers "F.Cu" "B.Cu") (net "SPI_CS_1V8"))
 (segment (start 126 28.7375) (end 126 17.5) (width 0.4) (layer "B.Cu") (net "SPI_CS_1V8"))
 (segment (start 126 21.5) (end 127.5 21.5) (width 0.2) (layer "F.Cu") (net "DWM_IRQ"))
 (segment (start 117.1625 39.35) (end 118.8375 39.35) (width 0.2) (layer "F.Cu") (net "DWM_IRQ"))
 (segment (start 90.25 62.9) (end 88.75 62.9) (width 0.2) (layer "F.Cu") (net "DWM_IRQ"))
 (segment (start 117.1625 39.35) (end 90.25 39.35) (width 0.2) (layer "F.Cu") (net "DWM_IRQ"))
 (segment (start 118.8375 39.35) (end 126 39.35) (width 0.2) (layer "F.Cu") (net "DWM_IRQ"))
 (via (at 126 39.35) (size 0.6) (drill 0.3) (layers "F.Cu" "B.Cu") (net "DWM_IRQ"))
 (via (at 90.25 39.35) (size 0.6) (drill 0.3) (layers "F.Cu" "B.Cu") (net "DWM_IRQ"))
 (via (at 126 21.5) (size 0.6) (drill 0.3) (layers "F.Cu" "B.Cu") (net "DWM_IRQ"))
 (via (at 90.25 62.9) (size 0.6) (drill 0.3) (layers "F.Cu" "B.Cu") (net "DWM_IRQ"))
 (segment (start 90.25 39.35) (end 90.25 62.9) (width 0.2) (layer "B.Cu") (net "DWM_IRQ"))
 (segment (start 126 39.35) (end 126 21.5) (width 0.2) (layer "B.Cu") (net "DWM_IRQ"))
 (segment (start 152 16) (end 144 16) (width 0.35) (layer "F.Cu") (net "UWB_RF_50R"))
 (segment (start 144 23.5) (end 142.5 23.5) (width 0.35) (layer "F.Cu") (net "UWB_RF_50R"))
 (via (at 144 16) (size 0.6) (drill 0.3) (layers "F.Cu" "B.Cu") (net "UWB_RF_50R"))
 (via (at 144 23.5) (size 0.6) (drill 0.3) (layers "F.Cu" "B.Cu") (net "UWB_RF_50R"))
 (segment (start 144 16) (end 144 23.5) (width 0.35) (layer "B.Cu") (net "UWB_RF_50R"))
 (segment (start 87.25 64.17) (end 88.75 64.17) (width 0.3) (layer "F.Cu") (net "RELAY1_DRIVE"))
 (segment (start 35.16 76) (end 87.25 76) (width 0.3) (layer "F.Cu") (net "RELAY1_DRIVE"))
 (segment (start 33.66 76) (end 35.16 76) (width 0.3) (layer "F.Cu") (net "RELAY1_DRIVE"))
 (segment (start 31.0625 61.05) (end 33.66 61.05) (width 0.3) (layer "F.Cu") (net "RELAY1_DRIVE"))
 (via (at 33.66 76) (size 0.6) (drill 0.3) (layers "F.Cu" "B.Cu") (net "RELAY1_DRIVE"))
 (via (at 87.25 64.17) (size 0.6) (drill 0.3) (layers "F.Cu" "B.Cu") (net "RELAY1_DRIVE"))
 (via (at 87.25 76) (size 0.6) (drill 0.3) (layers "F.Cu" "B.Cu") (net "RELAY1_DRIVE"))
 (via (at 33.66 61.05) (size 0.6) (drill 0.3) (layers "F.Cu" "B.Cu") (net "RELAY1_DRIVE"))
 (segment (start 87.25 76) (end 87.25 64.17) (width 0.3) (layer "B.Cu") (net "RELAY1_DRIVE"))
 (segment (start 33.66 61.05) (end 33.66 76) (width 0.3) (layer "B.Cu") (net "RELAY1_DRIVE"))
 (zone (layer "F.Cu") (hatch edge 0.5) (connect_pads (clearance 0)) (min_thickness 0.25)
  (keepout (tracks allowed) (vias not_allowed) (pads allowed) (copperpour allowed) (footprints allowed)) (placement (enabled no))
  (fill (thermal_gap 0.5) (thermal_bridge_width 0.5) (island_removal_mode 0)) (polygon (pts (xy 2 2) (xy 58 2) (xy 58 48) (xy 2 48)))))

